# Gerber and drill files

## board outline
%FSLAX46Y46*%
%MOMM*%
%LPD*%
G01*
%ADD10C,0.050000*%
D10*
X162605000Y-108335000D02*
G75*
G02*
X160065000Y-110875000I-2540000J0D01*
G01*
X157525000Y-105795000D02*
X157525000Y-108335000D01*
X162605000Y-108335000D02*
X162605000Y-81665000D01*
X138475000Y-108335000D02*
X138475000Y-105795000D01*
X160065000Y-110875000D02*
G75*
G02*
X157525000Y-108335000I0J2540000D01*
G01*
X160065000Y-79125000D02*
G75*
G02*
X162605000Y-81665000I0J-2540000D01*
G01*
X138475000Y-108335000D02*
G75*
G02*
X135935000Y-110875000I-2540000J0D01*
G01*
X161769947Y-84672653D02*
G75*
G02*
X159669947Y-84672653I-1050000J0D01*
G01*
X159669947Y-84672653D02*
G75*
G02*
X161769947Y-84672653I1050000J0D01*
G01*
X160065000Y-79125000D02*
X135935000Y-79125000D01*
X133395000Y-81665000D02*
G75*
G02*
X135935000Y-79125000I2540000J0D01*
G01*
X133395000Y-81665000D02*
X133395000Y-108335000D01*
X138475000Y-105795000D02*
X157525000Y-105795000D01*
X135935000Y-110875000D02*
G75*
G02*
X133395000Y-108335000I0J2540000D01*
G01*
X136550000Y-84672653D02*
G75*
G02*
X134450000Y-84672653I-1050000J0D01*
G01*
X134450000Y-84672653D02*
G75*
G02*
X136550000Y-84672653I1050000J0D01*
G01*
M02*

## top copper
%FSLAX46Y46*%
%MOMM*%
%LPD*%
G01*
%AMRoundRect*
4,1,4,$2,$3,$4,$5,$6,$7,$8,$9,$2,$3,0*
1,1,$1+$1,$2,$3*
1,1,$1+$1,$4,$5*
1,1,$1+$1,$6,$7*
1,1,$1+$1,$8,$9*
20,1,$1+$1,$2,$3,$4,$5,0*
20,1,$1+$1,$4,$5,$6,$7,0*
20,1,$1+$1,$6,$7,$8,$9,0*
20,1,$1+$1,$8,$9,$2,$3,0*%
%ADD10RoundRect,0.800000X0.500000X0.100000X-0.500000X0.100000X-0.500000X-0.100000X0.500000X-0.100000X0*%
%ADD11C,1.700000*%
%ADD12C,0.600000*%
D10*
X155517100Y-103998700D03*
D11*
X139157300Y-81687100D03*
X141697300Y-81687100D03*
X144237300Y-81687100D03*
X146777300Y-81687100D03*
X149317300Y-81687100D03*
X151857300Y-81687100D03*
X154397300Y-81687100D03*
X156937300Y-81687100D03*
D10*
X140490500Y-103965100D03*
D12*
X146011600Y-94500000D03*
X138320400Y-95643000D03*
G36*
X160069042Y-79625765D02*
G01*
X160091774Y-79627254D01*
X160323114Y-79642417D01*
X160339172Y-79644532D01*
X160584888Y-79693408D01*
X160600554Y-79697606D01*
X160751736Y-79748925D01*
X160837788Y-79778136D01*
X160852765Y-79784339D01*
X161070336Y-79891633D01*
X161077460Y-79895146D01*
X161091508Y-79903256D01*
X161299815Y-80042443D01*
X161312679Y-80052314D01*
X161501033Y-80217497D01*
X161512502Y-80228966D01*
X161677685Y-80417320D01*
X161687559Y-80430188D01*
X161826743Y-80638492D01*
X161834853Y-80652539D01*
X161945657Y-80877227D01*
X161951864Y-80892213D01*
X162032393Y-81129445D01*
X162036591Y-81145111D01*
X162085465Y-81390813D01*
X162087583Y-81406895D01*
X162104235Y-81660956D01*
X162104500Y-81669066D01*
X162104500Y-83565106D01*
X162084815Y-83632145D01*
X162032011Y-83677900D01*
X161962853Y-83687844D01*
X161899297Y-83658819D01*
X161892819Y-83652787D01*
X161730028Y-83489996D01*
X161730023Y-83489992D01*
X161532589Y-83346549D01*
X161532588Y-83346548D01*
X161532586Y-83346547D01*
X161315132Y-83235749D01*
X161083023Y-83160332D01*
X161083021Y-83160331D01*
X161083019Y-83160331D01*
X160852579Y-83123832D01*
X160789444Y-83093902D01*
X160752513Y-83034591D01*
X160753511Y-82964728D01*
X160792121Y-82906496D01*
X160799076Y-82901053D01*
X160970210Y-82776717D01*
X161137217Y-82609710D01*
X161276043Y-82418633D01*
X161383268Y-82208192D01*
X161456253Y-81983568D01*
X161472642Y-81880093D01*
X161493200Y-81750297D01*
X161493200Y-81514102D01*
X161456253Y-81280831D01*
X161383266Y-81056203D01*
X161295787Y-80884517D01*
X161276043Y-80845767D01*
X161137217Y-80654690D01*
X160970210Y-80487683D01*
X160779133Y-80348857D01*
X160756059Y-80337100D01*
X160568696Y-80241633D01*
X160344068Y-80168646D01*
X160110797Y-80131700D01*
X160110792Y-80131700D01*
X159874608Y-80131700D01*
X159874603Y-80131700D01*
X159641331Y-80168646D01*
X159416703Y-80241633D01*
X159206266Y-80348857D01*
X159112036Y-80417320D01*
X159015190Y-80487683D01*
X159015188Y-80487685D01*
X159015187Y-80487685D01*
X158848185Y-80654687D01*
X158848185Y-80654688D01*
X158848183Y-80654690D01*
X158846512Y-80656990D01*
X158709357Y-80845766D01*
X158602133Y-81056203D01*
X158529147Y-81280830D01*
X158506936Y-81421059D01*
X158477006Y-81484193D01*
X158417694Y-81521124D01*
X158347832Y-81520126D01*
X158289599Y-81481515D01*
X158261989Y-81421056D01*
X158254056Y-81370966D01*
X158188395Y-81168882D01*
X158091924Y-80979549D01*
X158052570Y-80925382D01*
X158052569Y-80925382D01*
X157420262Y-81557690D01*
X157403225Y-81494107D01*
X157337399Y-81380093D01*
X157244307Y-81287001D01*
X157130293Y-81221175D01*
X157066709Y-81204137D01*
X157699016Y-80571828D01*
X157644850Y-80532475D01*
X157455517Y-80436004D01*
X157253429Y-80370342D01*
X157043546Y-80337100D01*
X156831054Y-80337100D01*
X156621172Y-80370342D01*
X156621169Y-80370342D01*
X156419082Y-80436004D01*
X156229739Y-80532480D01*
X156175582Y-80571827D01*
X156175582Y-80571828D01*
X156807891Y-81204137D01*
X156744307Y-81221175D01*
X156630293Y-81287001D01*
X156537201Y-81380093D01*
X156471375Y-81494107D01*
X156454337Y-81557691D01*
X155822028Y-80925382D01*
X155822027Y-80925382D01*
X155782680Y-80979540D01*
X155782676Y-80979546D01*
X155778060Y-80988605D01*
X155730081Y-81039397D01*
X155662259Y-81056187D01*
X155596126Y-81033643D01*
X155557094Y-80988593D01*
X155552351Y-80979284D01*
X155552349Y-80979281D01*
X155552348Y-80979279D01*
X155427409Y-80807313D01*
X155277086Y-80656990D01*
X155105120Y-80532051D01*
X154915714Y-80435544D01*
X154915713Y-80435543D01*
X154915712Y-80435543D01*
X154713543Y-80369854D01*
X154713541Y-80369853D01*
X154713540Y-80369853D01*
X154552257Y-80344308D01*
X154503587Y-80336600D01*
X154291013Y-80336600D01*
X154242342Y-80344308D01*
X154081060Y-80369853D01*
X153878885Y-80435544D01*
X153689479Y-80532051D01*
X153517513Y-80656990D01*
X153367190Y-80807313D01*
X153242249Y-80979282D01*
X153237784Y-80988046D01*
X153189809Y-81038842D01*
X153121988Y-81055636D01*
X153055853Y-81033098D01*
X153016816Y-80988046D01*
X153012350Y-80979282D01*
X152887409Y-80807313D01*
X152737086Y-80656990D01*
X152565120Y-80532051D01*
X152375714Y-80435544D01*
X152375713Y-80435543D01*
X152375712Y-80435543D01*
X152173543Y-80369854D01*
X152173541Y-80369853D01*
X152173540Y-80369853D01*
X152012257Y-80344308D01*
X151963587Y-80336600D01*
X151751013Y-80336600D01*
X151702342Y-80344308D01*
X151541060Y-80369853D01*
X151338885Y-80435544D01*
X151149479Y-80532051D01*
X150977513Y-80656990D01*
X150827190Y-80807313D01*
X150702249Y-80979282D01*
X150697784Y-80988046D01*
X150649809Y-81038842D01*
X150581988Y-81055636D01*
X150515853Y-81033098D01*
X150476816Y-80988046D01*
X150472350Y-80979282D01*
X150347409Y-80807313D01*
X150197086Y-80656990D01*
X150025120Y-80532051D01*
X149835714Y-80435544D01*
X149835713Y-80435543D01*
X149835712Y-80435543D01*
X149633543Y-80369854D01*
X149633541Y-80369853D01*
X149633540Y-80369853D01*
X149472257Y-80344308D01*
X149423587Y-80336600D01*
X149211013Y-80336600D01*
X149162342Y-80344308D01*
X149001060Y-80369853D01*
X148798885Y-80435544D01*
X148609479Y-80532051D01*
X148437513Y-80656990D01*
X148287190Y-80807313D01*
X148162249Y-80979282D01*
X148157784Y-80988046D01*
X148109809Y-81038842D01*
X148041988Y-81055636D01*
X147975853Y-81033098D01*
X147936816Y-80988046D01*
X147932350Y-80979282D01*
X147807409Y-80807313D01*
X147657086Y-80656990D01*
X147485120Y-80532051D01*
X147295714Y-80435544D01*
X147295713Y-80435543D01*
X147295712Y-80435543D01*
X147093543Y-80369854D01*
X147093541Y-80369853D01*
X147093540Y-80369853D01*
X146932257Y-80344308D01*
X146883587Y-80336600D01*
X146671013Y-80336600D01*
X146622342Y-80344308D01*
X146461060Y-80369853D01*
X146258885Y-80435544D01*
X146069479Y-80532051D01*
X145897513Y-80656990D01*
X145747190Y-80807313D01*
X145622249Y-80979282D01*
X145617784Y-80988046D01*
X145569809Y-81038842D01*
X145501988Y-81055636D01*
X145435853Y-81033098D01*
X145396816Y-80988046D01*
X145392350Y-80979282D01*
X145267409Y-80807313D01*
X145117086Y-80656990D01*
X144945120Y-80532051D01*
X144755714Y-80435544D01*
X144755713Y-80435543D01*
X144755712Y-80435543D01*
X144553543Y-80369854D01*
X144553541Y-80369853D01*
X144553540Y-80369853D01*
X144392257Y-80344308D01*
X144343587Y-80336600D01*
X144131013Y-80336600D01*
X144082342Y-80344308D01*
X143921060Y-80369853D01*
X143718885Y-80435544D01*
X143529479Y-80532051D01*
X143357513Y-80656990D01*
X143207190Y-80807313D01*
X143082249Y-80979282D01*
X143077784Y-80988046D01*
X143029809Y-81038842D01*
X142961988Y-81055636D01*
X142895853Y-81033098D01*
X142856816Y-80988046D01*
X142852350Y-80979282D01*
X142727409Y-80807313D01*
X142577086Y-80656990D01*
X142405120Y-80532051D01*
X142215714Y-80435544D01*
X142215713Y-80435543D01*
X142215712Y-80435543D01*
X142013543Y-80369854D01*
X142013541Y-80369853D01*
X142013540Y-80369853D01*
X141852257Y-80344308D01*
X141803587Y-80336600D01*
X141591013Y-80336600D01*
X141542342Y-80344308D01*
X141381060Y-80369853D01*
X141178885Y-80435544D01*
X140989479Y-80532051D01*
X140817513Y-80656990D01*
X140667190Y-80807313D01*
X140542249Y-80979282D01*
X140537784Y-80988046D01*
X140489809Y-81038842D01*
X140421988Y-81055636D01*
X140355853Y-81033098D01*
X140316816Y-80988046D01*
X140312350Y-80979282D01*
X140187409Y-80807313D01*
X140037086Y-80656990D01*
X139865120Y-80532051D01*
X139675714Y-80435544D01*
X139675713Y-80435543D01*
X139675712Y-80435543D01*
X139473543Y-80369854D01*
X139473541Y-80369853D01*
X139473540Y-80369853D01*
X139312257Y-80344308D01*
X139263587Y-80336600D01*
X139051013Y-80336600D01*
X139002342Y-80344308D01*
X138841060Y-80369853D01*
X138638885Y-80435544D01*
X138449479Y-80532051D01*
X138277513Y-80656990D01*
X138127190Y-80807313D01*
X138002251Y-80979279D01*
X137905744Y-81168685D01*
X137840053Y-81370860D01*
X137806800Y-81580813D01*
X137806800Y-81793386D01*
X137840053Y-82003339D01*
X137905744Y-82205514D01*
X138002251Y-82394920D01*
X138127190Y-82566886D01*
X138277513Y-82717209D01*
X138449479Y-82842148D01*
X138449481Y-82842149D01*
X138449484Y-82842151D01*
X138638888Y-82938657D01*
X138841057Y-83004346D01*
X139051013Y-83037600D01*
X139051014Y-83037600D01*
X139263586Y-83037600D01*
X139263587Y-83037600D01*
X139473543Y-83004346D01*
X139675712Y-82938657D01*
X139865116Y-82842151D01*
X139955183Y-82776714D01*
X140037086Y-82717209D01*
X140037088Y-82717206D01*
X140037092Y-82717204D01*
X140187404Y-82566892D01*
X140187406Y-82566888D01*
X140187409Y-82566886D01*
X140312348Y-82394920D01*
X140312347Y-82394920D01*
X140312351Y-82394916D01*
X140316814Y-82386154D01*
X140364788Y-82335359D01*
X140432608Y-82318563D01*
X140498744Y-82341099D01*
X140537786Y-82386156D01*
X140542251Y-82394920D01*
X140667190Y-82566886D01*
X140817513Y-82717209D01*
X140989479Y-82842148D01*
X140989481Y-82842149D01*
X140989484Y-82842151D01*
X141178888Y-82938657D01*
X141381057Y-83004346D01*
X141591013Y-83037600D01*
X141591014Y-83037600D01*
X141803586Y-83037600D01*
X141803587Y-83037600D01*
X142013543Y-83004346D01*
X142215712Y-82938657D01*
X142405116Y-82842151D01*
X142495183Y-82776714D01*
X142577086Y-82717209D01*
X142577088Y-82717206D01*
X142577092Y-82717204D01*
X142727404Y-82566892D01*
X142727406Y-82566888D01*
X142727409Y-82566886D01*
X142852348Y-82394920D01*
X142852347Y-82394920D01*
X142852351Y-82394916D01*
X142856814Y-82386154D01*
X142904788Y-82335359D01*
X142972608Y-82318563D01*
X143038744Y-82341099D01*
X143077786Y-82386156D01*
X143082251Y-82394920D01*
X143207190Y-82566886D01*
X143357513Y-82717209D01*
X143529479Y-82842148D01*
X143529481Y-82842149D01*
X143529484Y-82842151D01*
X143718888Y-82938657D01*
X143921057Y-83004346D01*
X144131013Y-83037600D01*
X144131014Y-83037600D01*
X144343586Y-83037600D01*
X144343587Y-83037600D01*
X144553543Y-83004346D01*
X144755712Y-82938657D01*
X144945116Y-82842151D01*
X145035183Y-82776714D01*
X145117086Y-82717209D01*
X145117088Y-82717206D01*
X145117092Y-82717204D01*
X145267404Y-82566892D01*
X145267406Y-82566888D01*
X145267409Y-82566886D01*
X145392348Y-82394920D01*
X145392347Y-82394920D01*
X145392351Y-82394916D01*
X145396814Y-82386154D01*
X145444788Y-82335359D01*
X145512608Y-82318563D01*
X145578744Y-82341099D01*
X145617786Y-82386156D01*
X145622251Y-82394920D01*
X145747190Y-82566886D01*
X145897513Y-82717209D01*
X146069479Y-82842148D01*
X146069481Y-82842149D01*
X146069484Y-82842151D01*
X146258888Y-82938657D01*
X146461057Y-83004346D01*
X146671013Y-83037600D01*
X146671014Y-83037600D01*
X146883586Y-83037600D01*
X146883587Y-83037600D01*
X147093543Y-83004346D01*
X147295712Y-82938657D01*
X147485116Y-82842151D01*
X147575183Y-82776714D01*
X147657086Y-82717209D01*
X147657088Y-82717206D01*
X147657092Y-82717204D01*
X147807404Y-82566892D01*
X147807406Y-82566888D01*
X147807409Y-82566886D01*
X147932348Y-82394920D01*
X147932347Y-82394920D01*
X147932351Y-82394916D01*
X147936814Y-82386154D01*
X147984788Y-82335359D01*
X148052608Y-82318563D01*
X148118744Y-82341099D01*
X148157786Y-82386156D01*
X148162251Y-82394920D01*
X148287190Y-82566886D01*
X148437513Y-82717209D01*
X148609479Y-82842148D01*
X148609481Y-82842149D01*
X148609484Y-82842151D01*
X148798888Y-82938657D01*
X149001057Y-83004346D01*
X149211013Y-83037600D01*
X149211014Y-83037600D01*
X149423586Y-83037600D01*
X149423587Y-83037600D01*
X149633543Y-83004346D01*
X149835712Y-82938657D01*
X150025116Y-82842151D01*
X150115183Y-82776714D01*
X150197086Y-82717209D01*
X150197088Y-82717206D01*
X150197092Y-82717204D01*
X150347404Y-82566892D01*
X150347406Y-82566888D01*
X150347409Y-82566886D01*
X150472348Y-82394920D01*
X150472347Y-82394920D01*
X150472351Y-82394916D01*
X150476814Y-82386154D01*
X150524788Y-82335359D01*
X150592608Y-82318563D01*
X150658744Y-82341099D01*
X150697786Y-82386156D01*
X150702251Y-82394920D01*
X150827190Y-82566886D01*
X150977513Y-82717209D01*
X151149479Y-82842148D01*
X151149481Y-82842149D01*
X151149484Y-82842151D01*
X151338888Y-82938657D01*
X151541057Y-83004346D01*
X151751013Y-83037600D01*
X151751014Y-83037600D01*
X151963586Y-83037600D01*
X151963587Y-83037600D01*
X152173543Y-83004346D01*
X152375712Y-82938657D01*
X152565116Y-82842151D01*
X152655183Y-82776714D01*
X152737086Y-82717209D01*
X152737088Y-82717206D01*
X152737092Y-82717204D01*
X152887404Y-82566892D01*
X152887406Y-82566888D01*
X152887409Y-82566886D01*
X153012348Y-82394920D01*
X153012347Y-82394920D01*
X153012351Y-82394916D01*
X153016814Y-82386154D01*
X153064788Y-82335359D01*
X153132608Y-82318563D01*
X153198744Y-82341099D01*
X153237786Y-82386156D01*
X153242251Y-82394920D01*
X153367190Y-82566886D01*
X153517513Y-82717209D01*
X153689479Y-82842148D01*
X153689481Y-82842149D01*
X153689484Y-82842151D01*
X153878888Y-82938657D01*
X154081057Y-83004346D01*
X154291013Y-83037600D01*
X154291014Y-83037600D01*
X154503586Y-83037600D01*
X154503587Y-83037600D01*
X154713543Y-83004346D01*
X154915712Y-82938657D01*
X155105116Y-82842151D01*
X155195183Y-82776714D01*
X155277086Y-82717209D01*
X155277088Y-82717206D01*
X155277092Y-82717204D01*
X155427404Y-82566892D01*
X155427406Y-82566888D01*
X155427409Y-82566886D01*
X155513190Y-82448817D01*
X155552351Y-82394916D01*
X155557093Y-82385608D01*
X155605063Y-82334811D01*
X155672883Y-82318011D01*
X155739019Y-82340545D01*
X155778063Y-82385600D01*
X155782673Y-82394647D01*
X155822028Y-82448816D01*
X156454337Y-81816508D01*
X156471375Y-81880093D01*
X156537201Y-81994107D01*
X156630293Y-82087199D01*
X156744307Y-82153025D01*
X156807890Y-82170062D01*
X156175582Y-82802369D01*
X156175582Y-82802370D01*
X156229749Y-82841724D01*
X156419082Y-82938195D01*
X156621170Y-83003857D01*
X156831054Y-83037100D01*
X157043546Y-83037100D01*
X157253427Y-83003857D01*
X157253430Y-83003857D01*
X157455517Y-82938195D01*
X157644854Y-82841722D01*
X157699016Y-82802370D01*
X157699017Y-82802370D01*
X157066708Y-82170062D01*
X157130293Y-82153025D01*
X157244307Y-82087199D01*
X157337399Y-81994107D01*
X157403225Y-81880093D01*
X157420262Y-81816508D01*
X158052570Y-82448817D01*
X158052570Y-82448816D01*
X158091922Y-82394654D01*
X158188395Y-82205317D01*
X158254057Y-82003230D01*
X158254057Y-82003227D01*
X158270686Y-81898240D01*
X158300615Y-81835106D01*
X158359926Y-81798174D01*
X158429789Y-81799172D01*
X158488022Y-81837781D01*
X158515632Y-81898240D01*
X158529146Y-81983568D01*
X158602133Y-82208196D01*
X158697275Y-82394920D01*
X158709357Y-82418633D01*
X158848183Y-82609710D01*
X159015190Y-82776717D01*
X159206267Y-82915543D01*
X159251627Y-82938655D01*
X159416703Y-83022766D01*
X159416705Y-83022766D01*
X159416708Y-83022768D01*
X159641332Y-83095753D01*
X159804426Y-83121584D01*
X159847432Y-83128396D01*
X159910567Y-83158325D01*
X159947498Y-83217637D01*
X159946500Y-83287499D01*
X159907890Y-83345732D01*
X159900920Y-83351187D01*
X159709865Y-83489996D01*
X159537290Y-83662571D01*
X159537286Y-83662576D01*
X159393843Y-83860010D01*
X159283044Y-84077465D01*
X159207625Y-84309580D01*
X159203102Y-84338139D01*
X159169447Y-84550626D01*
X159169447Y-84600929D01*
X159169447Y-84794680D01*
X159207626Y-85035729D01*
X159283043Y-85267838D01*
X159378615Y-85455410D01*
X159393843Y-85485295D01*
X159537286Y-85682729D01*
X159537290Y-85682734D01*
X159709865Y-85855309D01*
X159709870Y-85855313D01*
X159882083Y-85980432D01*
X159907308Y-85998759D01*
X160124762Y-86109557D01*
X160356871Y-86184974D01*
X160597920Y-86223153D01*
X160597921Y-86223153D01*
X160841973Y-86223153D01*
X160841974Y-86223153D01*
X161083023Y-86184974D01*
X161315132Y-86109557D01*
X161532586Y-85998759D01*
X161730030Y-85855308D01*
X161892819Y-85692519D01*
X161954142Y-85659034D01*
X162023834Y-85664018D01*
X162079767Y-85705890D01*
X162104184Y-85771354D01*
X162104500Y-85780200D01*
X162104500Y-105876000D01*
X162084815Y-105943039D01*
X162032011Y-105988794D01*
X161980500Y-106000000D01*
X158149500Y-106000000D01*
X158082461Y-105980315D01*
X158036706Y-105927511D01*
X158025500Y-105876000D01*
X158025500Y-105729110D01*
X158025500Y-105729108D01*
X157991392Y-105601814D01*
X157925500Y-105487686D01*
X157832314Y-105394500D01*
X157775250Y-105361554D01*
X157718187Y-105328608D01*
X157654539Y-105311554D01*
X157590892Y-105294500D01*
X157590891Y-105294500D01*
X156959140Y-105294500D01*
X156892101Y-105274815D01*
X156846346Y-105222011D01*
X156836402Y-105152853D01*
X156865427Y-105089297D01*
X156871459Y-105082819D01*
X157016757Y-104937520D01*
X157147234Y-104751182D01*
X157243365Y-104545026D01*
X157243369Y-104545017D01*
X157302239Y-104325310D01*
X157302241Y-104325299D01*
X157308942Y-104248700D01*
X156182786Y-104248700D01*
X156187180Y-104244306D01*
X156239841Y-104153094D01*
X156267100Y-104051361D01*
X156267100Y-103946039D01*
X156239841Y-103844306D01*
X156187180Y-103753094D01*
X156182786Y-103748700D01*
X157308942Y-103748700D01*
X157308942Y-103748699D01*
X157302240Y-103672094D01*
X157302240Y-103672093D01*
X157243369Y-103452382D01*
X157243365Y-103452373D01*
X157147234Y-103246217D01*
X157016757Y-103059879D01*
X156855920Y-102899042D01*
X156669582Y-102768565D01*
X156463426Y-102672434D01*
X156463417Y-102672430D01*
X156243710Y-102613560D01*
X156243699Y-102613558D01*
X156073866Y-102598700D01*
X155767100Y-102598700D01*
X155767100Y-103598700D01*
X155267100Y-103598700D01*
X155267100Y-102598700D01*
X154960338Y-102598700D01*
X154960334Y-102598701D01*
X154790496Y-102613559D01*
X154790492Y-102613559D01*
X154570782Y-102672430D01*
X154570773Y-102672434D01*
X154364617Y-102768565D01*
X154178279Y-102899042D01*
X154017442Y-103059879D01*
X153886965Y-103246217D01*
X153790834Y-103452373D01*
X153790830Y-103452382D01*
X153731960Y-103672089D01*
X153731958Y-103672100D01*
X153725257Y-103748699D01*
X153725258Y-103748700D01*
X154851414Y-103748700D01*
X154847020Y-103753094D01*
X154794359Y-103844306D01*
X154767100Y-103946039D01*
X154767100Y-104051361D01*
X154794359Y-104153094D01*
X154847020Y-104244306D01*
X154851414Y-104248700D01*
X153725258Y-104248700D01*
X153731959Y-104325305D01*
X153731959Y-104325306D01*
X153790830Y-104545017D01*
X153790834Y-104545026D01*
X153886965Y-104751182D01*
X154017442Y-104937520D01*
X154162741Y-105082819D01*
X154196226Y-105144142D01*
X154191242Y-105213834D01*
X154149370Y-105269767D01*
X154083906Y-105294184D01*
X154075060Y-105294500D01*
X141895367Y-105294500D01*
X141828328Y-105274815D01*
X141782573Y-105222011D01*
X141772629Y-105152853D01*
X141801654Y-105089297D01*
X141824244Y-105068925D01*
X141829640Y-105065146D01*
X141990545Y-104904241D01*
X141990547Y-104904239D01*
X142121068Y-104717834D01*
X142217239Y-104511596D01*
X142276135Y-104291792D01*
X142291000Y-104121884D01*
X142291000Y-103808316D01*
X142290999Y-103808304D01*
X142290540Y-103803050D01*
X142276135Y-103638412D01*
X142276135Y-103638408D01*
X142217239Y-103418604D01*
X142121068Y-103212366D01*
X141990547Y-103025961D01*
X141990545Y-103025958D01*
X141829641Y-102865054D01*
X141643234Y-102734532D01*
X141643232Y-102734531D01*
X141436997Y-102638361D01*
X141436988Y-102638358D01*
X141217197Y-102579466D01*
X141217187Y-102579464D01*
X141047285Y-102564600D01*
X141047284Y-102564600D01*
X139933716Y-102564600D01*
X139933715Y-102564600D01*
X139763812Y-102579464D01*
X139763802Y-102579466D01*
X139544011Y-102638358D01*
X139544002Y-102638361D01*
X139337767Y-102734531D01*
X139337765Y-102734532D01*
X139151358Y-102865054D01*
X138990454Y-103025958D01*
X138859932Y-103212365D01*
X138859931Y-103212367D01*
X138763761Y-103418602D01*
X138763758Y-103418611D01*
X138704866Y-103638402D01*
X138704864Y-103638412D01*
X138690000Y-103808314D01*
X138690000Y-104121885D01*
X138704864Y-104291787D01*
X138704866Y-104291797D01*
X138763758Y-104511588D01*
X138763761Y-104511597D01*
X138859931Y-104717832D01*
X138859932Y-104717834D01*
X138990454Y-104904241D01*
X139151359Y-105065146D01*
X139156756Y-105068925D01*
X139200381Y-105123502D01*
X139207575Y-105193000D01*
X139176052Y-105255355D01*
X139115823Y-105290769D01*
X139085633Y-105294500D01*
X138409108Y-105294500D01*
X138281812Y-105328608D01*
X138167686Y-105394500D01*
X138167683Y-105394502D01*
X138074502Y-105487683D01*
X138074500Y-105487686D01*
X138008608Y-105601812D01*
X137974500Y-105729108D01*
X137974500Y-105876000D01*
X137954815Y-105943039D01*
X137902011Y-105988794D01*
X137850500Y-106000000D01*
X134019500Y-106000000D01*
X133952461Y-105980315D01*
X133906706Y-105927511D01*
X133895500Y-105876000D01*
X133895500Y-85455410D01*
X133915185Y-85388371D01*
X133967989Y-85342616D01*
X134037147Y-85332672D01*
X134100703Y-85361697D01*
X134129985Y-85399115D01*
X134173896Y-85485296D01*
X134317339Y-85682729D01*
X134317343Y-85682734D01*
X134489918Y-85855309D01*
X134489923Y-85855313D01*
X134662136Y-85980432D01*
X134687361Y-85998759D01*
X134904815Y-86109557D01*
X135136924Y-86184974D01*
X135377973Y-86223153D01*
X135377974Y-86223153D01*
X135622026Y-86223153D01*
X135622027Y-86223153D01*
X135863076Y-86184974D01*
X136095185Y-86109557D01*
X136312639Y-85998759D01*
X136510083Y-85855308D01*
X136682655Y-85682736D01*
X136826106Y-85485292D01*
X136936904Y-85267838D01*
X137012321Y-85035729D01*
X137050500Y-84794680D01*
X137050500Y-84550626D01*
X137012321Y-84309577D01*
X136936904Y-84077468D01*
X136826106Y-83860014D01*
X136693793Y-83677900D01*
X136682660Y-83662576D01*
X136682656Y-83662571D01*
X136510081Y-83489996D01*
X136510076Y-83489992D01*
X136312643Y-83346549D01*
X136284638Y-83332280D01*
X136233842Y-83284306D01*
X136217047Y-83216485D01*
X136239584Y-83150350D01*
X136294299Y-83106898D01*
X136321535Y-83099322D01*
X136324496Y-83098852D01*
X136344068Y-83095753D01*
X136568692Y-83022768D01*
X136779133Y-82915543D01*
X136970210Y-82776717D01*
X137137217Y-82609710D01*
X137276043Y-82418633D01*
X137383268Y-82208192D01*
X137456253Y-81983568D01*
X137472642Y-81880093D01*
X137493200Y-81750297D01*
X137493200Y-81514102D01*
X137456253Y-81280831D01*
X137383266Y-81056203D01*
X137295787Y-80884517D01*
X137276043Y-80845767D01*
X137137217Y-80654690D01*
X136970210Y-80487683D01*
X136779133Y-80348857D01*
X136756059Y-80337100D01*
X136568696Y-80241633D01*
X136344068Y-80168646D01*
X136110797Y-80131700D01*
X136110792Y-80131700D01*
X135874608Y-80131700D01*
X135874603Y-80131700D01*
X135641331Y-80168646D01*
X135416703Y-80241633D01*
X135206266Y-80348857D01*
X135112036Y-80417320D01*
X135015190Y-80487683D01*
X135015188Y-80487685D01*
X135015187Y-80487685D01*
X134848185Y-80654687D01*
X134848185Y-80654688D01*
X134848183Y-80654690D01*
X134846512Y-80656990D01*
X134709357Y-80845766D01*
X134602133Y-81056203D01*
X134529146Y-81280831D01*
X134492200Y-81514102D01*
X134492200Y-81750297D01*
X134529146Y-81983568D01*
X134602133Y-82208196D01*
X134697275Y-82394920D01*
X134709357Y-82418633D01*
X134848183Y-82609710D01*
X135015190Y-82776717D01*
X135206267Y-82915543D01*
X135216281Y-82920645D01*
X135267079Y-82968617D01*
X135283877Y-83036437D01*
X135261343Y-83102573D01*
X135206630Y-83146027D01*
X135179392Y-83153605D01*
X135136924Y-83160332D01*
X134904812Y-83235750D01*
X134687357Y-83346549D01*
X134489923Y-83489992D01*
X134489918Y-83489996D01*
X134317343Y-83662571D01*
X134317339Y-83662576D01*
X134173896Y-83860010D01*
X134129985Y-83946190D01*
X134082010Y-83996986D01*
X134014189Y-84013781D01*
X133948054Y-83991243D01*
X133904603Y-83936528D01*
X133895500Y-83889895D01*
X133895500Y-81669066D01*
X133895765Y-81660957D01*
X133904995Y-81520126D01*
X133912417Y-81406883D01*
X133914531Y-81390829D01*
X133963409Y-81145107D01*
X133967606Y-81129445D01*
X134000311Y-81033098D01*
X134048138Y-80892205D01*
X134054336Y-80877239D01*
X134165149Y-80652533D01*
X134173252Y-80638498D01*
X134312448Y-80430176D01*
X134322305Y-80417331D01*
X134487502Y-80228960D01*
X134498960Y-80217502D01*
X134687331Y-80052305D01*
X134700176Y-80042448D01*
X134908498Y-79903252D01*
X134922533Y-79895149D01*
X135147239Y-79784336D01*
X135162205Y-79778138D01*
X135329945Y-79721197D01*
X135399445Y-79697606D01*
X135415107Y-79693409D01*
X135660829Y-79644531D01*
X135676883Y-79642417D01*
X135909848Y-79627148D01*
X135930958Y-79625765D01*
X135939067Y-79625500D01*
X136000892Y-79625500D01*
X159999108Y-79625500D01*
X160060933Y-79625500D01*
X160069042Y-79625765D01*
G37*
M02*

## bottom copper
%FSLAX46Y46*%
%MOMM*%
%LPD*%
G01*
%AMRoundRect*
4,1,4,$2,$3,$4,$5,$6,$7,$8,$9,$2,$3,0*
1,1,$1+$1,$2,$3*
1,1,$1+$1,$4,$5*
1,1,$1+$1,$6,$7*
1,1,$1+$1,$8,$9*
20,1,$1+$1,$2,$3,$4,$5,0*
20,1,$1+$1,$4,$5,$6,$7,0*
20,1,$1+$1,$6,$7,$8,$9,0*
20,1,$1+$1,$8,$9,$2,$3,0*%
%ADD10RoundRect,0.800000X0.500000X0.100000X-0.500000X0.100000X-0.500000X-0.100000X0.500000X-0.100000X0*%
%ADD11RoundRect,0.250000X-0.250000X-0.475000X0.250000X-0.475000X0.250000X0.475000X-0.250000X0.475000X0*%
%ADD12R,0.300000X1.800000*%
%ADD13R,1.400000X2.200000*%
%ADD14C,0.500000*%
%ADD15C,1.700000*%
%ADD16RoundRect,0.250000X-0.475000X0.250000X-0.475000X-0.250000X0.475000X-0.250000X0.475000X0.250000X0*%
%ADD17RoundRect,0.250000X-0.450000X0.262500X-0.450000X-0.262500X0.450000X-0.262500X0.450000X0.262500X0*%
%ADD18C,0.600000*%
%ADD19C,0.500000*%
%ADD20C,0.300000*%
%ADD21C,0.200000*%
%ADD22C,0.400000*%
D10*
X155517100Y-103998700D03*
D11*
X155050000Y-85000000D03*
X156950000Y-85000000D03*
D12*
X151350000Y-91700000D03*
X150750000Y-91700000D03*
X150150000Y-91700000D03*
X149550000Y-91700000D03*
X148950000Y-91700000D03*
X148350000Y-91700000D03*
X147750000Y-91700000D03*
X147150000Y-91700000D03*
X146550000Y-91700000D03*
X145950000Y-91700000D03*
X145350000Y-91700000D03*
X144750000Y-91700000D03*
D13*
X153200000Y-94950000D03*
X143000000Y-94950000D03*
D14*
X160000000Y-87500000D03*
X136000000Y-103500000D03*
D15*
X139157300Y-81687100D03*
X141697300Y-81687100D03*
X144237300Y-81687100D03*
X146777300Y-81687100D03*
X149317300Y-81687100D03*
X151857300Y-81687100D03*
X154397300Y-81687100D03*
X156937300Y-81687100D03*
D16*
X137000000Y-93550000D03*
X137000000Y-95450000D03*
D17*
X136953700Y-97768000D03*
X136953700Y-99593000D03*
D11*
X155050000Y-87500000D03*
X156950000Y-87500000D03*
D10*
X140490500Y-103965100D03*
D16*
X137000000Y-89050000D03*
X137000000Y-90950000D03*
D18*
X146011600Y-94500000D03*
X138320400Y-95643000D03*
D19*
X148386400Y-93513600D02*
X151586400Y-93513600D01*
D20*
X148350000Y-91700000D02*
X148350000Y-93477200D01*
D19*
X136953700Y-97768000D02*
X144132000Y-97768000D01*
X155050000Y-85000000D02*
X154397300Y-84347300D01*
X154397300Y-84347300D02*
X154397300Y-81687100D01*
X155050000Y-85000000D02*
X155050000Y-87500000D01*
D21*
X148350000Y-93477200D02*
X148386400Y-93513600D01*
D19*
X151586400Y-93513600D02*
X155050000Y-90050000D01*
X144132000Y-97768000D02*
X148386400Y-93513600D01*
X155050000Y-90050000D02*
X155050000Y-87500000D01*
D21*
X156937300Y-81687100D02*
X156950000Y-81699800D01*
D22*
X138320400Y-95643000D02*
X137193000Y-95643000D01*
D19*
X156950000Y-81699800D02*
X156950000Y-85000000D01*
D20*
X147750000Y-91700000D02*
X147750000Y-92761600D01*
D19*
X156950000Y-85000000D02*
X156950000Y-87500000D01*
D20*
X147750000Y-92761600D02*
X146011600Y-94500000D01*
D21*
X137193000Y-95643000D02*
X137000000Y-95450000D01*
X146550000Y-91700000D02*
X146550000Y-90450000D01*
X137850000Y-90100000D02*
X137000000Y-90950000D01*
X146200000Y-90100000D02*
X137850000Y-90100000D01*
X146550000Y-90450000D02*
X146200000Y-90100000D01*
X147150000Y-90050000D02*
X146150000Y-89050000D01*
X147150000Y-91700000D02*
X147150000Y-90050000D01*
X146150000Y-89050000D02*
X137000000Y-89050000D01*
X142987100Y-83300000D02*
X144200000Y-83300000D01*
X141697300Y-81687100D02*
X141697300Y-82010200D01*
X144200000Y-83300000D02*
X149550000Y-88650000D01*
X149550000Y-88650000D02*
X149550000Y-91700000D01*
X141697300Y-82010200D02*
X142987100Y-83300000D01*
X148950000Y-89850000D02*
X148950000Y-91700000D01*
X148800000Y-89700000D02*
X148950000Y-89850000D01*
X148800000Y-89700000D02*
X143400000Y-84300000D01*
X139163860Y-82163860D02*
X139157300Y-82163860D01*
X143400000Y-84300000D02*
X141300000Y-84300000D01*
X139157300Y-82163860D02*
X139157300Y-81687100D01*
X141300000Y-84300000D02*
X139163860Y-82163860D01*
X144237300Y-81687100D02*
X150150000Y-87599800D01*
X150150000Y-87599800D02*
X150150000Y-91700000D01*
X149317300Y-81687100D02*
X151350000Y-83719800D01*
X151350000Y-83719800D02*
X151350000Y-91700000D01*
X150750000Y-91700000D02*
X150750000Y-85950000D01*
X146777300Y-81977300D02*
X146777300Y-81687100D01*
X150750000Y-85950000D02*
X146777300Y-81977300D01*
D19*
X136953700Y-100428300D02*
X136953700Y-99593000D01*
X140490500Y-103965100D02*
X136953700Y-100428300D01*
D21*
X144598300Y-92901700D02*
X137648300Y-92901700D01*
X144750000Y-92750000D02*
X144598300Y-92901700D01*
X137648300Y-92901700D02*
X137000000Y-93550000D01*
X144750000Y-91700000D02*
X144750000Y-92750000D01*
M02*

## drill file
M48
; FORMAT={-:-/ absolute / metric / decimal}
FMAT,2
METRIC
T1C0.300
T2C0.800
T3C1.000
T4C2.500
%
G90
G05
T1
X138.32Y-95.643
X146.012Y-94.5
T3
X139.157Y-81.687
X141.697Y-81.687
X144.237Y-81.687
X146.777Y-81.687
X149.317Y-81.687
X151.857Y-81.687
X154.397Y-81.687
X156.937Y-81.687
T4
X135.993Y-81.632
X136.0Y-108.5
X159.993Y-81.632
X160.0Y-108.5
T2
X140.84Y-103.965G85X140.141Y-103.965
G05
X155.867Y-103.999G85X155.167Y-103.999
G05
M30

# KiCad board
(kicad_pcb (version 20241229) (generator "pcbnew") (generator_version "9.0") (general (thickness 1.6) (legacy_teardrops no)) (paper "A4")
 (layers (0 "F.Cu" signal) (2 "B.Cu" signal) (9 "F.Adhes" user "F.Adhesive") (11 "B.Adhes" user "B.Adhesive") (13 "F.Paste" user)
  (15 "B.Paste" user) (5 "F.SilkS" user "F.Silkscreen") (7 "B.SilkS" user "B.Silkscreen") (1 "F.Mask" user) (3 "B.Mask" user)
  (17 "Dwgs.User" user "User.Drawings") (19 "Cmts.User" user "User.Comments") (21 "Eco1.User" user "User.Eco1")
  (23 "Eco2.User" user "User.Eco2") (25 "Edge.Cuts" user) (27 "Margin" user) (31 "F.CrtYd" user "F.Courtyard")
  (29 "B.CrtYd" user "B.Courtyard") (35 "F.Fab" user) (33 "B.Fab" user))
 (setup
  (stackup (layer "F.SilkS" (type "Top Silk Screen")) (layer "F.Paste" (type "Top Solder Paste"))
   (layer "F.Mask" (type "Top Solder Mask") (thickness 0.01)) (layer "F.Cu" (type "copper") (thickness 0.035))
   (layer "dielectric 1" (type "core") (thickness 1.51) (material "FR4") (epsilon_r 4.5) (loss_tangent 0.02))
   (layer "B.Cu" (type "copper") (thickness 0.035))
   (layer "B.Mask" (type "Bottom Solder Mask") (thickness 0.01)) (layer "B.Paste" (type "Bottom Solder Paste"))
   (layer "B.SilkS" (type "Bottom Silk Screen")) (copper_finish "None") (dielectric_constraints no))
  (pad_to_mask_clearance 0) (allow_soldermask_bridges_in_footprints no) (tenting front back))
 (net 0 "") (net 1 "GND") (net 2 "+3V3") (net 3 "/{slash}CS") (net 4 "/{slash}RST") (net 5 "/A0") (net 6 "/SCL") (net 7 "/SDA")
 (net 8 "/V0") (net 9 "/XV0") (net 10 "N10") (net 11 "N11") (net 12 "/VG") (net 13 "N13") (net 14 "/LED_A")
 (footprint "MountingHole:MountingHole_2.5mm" (layer "F.Cu") (at 160 108.5)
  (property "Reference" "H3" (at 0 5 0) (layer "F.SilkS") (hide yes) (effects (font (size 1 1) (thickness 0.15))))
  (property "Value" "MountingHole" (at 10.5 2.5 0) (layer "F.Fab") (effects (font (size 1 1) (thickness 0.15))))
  (pad "" np_thru_hole circle (at 0 0) (size 2.5 2.5) (drill 2.5) (layers "*.Cu" "*.Mask")))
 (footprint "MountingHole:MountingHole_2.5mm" (layer "F.Cu") (at 159.9927 81.6322)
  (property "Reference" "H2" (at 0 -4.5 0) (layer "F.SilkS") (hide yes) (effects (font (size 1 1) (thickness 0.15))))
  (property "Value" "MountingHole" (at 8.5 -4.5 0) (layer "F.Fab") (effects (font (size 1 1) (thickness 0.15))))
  (pad "" np_thru_hole circle (at 0 0) (size 2.5 2.5) (drill 2.5) (layers "*.Cu" "*.Mask")))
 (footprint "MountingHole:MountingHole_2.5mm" (layer "F.Cu") (at 135.9927 81.6322)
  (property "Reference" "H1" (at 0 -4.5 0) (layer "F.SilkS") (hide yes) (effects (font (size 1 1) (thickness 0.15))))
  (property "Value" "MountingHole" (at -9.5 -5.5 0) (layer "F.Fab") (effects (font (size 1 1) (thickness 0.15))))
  (pad "" np_thru_hole circle (at 0 0) (size 2.5 2.5) (drill 2.5) (layers "*.Cu" "*.Mask")))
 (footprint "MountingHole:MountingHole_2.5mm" (layer "F.Cu") (at 136 108.5)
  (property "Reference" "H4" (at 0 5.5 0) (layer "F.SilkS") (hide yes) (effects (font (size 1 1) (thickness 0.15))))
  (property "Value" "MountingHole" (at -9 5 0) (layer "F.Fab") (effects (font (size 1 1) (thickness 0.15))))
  (pad "" np_thru_hole circle (at 0 0) (size 2.5 2.5) (drill 2.5) (layers "*.Cu" "*.Mask")))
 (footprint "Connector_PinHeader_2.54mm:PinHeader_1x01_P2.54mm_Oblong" (layer "B.Cu") (at 155.5171 103.9987 180)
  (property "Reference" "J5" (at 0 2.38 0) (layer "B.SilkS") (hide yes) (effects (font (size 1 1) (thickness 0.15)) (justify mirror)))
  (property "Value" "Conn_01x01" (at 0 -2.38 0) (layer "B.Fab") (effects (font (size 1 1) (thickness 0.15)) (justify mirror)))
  (pad "1" thru_hole roundrect (at 0 0 180) (size 2.6 1.8) (drill oval 1.5 0.8) (layers "*.Cu" "*.Mask") (remove_unused_layers no)
   (roundrect_rratio 0.4444444444) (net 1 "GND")))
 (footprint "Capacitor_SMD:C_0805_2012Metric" (layer "B.Cu") (at 156 85)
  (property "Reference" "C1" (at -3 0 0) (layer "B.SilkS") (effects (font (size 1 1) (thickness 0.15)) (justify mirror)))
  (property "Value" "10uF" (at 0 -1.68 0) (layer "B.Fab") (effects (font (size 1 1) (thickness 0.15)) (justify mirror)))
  (pad "1" smd roundrect (at -0.95 0) (size 1 1.45) (layers "B.Cu" "B.Mask" "B.Paste") (roundrect_rratio 0.25) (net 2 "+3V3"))
  (pad "2" smd roundrect (at 0.95 0) (size 1 1.45) (layers "B.Cu" "B.Mask" "B.Paste") (roundrect_rratio 0.25) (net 1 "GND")))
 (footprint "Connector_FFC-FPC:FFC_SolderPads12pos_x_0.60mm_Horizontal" (layer "B.Cu") (at 148.5 93.55 180)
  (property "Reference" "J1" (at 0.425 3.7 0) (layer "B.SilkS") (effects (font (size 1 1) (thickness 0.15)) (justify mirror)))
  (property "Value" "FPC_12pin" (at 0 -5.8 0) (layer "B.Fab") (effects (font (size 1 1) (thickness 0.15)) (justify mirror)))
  (pad "1" smd rect (at -2.85 1.85 180) (size 0.3 1.8) (layers "B.Cu" "B.Mask" "B.Paste") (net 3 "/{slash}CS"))
  (pad "2" smd rect (at -2.25 1.85 180) (size 0.3 1.8) (layers "B.Cu" "B.Mask" "B.Paste") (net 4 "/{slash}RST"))
  (pad "3" smd rect (at -1.65 1.85 180) (size 0.3 1.8) (layers "B.Cu" "B.Mask" "B.Paste") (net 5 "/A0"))
  (pad "4" smd rect (at -1.05 1.85 180) (size 0.3 1.8) (layers "B.Cu" "B.Mask" "B.Paste") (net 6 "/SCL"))
  (pad "5" smd rect (at -0.45 1.85 180) (size 0.3 1.8) (layers "B.Cu" "B.Mask" "B.Paste") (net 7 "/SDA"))
  (pad "6" smd rect (at 0.15 1.85 180) (size 0.3 1.8) (layers "B.Cu" "B.Mask" "B.Paste") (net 2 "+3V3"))
  (pad "7" smd rect (at 0.75 1.85 180) (size 0.3 1.8) (layers "B.Cu" "B.Mask" "B.Paste") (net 1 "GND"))
  (pad "8" smd rect (at 1.35 1.85 180) (size 0.3 1.8) (layers "B.Cu" "B.Mask" "B.Paste") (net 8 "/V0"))
  (pad "9" smd rect (at 1.95 1.85 180) (size 0.3 1.8) (layers "B.Cu" "B.Mask" "B.Paste") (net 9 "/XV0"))
  (pad "10" smd rect (at 2.55 1.85 180) (size 0.3 1.8) (layers "B.Cu" "B.Mask" "B.Paste") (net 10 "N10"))
  (pad "11" smd rect (at 3.15 1.85 180) (size 0.3 1.8) (layers "B.Cu" "B.Mask" "B.Paste") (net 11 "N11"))
  (pad "12" smd rect (at 3.75 1.85 180) (size 0.3 1.8) (layers "B.Cu" "B.Mask" "B.Paste") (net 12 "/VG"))
  (pad "MP" smd rect (at -4.7 -1.4 180) (size 1.4 2.2) (layers "B.Cu" "B.Mask" "B.Paste"))
  (pad "MP" smd rect (at 5.5 -1.4 180) (size 1.4 2.2) (layers "B.Cu" "B.Mask" "B.Paste")))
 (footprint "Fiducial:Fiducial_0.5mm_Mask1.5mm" (layer "B.Cu") (at 160 87.5 180)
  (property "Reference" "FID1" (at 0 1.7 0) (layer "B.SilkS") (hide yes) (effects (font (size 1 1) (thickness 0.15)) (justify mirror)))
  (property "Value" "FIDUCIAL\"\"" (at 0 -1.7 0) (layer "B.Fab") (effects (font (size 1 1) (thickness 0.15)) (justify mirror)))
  (pad "" smd circle (at 0 0 180) (size 0.5 0.5) (layers "B.Cu" "B.Mask") (solder_mask_margin 0.5) (clearance 0.6)))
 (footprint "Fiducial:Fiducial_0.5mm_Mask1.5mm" (layer "B.Cu") (at 136 103.5 180)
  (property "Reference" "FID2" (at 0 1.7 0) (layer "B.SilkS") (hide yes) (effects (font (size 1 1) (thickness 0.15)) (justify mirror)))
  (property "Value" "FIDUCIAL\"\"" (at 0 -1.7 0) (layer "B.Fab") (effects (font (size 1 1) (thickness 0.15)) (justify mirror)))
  (pad "" smd circle (at 0 0 180) (size 0.5 0.5) (layers "B.Cu" "B.Mask") (solder_mask_margin 0.5) (clearance 0.6)))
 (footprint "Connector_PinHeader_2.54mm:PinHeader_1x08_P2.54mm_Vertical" (layer "B.Cu") (at 139.1573 81.6871 -90)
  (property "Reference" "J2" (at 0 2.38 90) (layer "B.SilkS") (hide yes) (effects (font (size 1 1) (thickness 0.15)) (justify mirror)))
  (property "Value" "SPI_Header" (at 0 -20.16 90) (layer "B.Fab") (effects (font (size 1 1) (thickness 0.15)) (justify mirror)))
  (pad "1" thru_hole circle (at 0 0 270) (size 1.7 1.7) (drill 1) (layers "*.Cu" "*.Mask") (remove_unused_layers no) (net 7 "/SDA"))
  (pad "2" thru_hole circle (at 0 -2.54 270) (size 1.7 1.7) (drill 1) (layers "*.Cu" "*.Mask") (remove_unused_layers no) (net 6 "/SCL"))
  (pad "3" thru_hole circle (at 0 -5.08 270) (size 1.7 1.7) (drill 1) (layers "*.Cu" "*.Mask") (remove_unused_layers no) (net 5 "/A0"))
  (pad "4" thru_hole circle (at 0 -7.62 270) (size 1.7 1.7) (drill 1) (layers "*.Cu" "*.Mask") (remove_unused_layers no)
   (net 4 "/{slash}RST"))
  (pad "5" thru_hole circle (at 0 -10.16 270) (size 1.7 1.7) (drill 1) (layers "*.Cu" "*.Mask") (remove_unused_layers no)
   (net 3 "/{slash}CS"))
  (pad "6" thru_hole circle (at 0 -12.7 270) (size 1.7 1.7) (drill 1) (layers "*.Cu" "*.Mask") (remove_unused_layers no) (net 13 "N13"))
  (pad "7" thru_hole circle (at 0 -15.24 270) (size 1.7 1.7) (drill 1) (layers "*.Cu" "*.Mask") (remove_unused_layers no) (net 2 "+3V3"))
  (pad "8" thru_hole circle (at 0 -17.78 270) (size 1.7 1.7) (drill 1) (layers "*.Cu" "*.Mask") (remove_unused_layers no) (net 1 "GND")))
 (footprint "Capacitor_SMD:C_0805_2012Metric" (layer "B.Cu") (at 137 94.5 -90)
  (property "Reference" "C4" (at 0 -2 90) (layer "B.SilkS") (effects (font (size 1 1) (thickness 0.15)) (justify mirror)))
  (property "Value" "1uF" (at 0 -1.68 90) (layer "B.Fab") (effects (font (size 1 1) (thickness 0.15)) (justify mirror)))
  (pad "1" smd roundrect (at -0.95 0 270) (size 1 1.45) (layers "B.Cu" "B.Mask" "B.Paste") (roundrect_rratio 0.25) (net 12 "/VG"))
  (pad "2" smd roundrect (at 0.95 0 270) (size 1 1.45) (layers "B.Cu" "B.Mask" "B.Paste") (roundrect_rratio 0.25) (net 1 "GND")))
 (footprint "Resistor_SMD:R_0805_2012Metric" (layer "B.Cu") (at 136.9537 98.6805 -90)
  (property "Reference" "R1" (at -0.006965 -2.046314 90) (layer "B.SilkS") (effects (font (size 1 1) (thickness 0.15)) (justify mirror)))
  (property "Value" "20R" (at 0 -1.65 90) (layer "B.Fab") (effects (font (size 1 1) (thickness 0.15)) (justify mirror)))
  (pad "1" smd roundrect (at -0.9125 0 270) (size 1.025 1.4) (layers "B.Cu" "B.Mask" "B.Paste") (roundrect_rratio 0.243902) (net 2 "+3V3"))
  (pad "2" smd roundrect (at 0.9125 0 270) (size 1.025 1.4) (layers "B.Cu" "B.Mask" "B.Paste") (roundrect_rratio 0.243902) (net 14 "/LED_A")))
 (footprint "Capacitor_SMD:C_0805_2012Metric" (layer "B.Cu") (at 156 87.5)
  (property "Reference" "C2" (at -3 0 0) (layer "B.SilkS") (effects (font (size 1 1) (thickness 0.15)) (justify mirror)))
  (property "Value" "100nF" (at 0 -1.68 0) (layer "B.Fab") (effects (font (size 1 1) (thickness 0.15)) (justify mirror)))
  (pad "1" smd roundrect (at -0.95 0) (size 1 1.45) (layers "B.Cu" "B.Mask" "B.Paste") (roundrect_rratio 0.25) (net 2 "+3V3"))
  (pad "2" smd roundrect (at 0.95 0) (size 1 1.45) (layers "B.Cu" "B.Mask" "B.Paste") (roundrect_rratio 0.25) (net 1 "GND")))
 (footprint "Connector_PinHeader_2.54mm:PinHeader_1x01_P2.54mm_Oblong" (layer "B.Cu") (at 140.4905 103.9651 180)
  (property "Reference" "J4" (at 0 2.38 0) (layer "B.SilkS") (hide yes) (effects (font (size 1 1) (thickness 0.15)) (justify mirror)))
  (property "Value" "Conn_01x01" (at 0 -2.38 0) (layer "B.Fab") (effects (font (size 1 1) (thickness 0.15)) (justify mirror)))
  (pad "1" thru_hole roundrect (at 0 0 180) (size 2.6 1.8) (drill oval 1.5 0.8) (layers "*.Cu" "*.Mask") (remove_unused_layers no)
   (roundrect_rratio 0.4444444444) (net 14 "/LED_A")))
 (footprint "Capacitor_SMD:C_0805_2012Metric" (layer "B.Cu") (at 137 90 -90)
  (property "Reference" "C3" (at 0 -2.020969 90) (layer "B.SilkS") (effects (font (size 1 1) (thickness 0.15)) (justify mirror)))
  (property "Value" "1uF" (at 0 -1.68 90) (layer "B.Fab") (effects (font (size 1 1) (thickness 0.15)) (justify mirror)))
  (pad "1" smd roundrect (at -0.95 0 270) (size 1 1.45) (layers "B.Cu" "B.Mask" "B.Paste") (roundrect_rratio 0.25) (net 8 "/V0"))
  (pad "2" smd roundrect (at 0.95 0 270) (size 1 1.45) (layers "B.Cu" "B.Mask" "B.Paste") (roundrect_rratio 0.25) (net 9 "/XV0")))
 (gr_arc (start 162.605 108.335) (mid 161.861051 110.131051) (end 160.065 110.875) (stroke (width 0.05) (type solid)) (layer "Edge.Cuts"))
 (gr_line (start 157.525 105.795) (end 157.525 108.335) (stroke (width 0.05) (type solid)) (layer "Edge.Cuts"))
 (gr_line (start 162.605 108.335) (end 162.605 81.665) (stroke (width 0.05) (type solid)) (layer "Edge.Cuts"))
 (gr_line (start 138.475 108.335) (end 138.475 105.795) (stroke (width 0.05) (type solid)) (layer "Edge.Cuts"))
 (gr_arc (start 160.065 110.875) (mid 158.268949 110.131051) (end 157.525 108.335) (stroke (width 0.05) (type solid)) (layer "Edge.Cuts"))
 (gr_arc (start 160.065 79.125) (mid 161.861051 79.868949) (end 162.605 81.665) (stroke (width 0.05) (type solid)) (layer "Edge.Cuts"))
 (gr_arc (start 138.475 108.335) (mid 137.731051 110.131051) (end 135.935 110.875) (stroke (width 0.05) (type solid)) (layer "Edge.Cuts"))
 (gr_circle (center 160.719947 84.672653) (end 161.769947 84.672653) (stroke (width 0.05) (type solid)) (fill no) (layer "Edge.Cuts"))
 (gr_line (start 160.065 79.125) (end 135.935 79.125) (stroke (width 0.05) (type solid)) (layer "Edge.Cuts"))
 (gr_arc (start 133.395 81.665) (mid 134.138949 79.868949) (end 135.935 79.125) (stroke (width 0.05) (type solid)) (layer "Edge.Cuts"))
 (gr_line (start 133.395 81.665) (end 133.395 108.335) (stroke (width 0.05) (type solid)) (layer "Edge.Cuts"))
 (gr_line (start 138.475 105.795) (end 157.525 105.795) (stroke (width 0.05) (type solid)) (layer "Edge.Cuts"))
 (gr_arc (start 135.935 110.875) (mid 134.138949 110.131051) (end 133.395 108.335) (stroke (width 0.05) (type solid)) (layer "Edge.Cuts"))
 (gr_circle (center 135.5 84.672653) (end 136.55 84.672653) (stroke (width 0.05) (type solid)) (fill no) (layer "Edge.Cuts"))
 (segment (start 148.3864 93.5136) (end 151.5864 93.5136) (width 0.5) (layer "B.Cu") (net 2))
 (segment (start 148.35 91.7) (end 148.35 93.4772) (width 0.3) (layer "B.Cu") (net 2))
 (segment (start 136.9537 97.768) (end 144.132 97.768) (width 0.5) (layer "B.Cu") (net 2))
 (segment (start 155.05 85) (end 154.3973 84.3473) (width 0.5) (layer "B.Cu") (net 2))
 (segment (start 154.3973 84.3473) (end 154.3973 81.6871) (width 0.5) (layer "B.Cu") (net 2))
 (segment (start 155.05 85) (end 155.05 87.5) (width 0.5) (layer "B.Cu") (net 2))
 (segment (start 148.35 93.4772) (end 148.3864 93.5136) (width 0.2) (layer "B.Cu") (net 2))
 (segment (start 151.5864 93.5136) (end 155.05 90.05) (width 0.5) (layer "B.Cu") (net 2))
 (segment (start 144.132 97.768) (end 148.3864 93.5136) (width 0.5) (layer "B.Cu") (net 2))
 (segment (start 155.05 90.05) (end 155.05 87.5) (width 0.5) (layer "B.Cu") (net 2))
 (via (at 146.0116 94.5) (size 0.6) (drill 0.3) (layers "F.Cu" "B.Cu") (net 1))
 (via (at 138.3204 95.643) (size 0.6) (drill 0.3) (layers "F.Cu" "B.Cu") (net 1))
 (segment (start 156.9373 81.6871) (end 156.95 81.6998) (width 0.2) (layer "B.Cu") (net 1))
 (segment (start 138.3204 95.643) (end 137.193 95.643) (width 0.4) (layer "B.Cu") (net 1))
 (segment (start 156.95 81.6998) (end 156.95 85) (width 0.5) (layer "B.Cu") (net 1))
 (segment (start 147.75 91.7) (end 147.75 92.7616) (width 0.3) (layer "B.Cu") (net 1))
 (segment (start 156.95 85) (end 156.95 87.5) (width 0.5) (layer "B.Cu") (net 1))
 (segment (start 147.75 92.7616) (end 146.0116 94.5) (width 0.3) (layer "B.Cu") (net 1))
 (segment (start 137.193 95.643) (end 137 95.45) (width 0.2) (layer "B.Cu") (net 1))
 (segment (start 146.55 91.7) (end 146.55 90.45) (width 0.2) (layer "B.Cu") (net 9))
 (segment (start 137.85 90.1) (end 137 90.95) (width 0.2) (layer "B.Cu") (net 9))
 (segment (start 146.2 90.1) (end 137.85 90.1) (width 0.2) (layer "B.Cu") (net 9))
 (segment (start 146.55 90.45) (end 146.2 90.1) (width 0.2) (layer "B.Cu") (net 9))
 (segment (start 147.15 90.05) (end 146.15 89.05) (width 0.2) (layer "B.Cu") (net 8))
 (segment (start 147.15 91.7) (end 147.15 90.05) (width 0.2) (layer "B.Cu") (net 8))
 (segment (start 146.15 89.05) (end 137 89.05) (width 0.2) (layer "B.Cu") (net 8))
 (segment (start 142.9871 83.3) (end 144.2 83.3) (width 0.2) (layer "B.Cu") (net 6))
 (segment (start 141.6973 81.6871) (end 141.6973 82.0102) (width 0.2) (layer "B.Cu") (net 6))
 (segment (start 144.2 83.3) (end 149.55 88.65) (width 0.2) (layer "B.Cu") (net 6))
 (segment (start 149.55 88.65) (end 149.55 91.7) (width 0.2) (layer "B.Cu") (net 6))
 (segment (start 141.6973 82.0102) (end 142.9871 83.3) (width 0.2) (layer "B.Cu") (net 6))
 (segment (start 148.95 89.85) (end 148.95 91.7) (width 0.2) (layer "B.Cu") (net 7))
 (segment (start 148.8 89.7) (end 148.95 89.85) (width 0.2) (layer "B.Cu") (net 7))
 (segment (start 148.8 89.7) (end 143.4 84.3) (width 0.2) (layer "B.Cu") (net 7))
 (segment (start 139.16386 82.16386) (end 139.1573 82.16386) (width 0.2) (layer "B.Cu") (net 7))
 (segment (start 143.4 84.3) (end 141.3 84.3) (width 0.2) (layer "B.Cu") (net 7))
 (segment (start 139.1573 82.16386) (end 139.1573 81.6871) (width 0.2) (layer "B.Cu") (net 7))
 (segment (start 141.3 84.3) (end 139.16386 82.16386) (width 0.2) (layer "B.Cu") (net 7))
 (segment (start 144.2373 81.6871) (end 150.15 87.5998) (width 0.2) (layer "B.Cu") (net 5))
 (segment (start 150.15 87.5998) (end 150.15 91.7) (width 0.2) (layer "B.Cu") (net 5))
 (segment (start 149.3173 81.6871) (end 151.35 83.7198) (width 0.2) (layer "B.Cu") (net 3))
 (segment (start 151.35 83.7198) (end 151.35 91.7) (width 0.2) (layer "B.Cu") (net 3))
 (segment (start 150.75 91.7) (end 150.75 85.95) (width 0.2) (layer "B.Cu") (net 4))
 (segment (start 146.7773 81.9773) (end 146.7773 81.6871) (width 0.2) (layer "B.Cu") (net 4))
 (segment (start 150.75 85.95) (end 146.7773 81.9773) (width 0.2) (layer "B.Cu") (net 4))
 (segment (start 136.9537 100.4283) (end 136.9537 99.593) (width 0.5) (layer "B.Cu") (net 14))
 (segment (start 140.4905 103.9651) (end 136.9537 100.4283) (width 0.5) (layer "B.Cu") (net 14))
 (segment (start 144.5983 92.9017) (end 137.6483 92.9017) (width 0.2) (layer "B.Cu") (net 12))
 (segment (start 144.75 92.75) (end 144.5983 92.9017) (width 0.2) (layer "B.Cu") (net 12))
 (segment (start 137.6483 92.9017) (end 137 93.55) (width 0.2) (layer "B.Cu") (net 12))
 (segment (start 144.75 91.7) (end 144.75 92.75) (width 0.2) (layer "B.Cu") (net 12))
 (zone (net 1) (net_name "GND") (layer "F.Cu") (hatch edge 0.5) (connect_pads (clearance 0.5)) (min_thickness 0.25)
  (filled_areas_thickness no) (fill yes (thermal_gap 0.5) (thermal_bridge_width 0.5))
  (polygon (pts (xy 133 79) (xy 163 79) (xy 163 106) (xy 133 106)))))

